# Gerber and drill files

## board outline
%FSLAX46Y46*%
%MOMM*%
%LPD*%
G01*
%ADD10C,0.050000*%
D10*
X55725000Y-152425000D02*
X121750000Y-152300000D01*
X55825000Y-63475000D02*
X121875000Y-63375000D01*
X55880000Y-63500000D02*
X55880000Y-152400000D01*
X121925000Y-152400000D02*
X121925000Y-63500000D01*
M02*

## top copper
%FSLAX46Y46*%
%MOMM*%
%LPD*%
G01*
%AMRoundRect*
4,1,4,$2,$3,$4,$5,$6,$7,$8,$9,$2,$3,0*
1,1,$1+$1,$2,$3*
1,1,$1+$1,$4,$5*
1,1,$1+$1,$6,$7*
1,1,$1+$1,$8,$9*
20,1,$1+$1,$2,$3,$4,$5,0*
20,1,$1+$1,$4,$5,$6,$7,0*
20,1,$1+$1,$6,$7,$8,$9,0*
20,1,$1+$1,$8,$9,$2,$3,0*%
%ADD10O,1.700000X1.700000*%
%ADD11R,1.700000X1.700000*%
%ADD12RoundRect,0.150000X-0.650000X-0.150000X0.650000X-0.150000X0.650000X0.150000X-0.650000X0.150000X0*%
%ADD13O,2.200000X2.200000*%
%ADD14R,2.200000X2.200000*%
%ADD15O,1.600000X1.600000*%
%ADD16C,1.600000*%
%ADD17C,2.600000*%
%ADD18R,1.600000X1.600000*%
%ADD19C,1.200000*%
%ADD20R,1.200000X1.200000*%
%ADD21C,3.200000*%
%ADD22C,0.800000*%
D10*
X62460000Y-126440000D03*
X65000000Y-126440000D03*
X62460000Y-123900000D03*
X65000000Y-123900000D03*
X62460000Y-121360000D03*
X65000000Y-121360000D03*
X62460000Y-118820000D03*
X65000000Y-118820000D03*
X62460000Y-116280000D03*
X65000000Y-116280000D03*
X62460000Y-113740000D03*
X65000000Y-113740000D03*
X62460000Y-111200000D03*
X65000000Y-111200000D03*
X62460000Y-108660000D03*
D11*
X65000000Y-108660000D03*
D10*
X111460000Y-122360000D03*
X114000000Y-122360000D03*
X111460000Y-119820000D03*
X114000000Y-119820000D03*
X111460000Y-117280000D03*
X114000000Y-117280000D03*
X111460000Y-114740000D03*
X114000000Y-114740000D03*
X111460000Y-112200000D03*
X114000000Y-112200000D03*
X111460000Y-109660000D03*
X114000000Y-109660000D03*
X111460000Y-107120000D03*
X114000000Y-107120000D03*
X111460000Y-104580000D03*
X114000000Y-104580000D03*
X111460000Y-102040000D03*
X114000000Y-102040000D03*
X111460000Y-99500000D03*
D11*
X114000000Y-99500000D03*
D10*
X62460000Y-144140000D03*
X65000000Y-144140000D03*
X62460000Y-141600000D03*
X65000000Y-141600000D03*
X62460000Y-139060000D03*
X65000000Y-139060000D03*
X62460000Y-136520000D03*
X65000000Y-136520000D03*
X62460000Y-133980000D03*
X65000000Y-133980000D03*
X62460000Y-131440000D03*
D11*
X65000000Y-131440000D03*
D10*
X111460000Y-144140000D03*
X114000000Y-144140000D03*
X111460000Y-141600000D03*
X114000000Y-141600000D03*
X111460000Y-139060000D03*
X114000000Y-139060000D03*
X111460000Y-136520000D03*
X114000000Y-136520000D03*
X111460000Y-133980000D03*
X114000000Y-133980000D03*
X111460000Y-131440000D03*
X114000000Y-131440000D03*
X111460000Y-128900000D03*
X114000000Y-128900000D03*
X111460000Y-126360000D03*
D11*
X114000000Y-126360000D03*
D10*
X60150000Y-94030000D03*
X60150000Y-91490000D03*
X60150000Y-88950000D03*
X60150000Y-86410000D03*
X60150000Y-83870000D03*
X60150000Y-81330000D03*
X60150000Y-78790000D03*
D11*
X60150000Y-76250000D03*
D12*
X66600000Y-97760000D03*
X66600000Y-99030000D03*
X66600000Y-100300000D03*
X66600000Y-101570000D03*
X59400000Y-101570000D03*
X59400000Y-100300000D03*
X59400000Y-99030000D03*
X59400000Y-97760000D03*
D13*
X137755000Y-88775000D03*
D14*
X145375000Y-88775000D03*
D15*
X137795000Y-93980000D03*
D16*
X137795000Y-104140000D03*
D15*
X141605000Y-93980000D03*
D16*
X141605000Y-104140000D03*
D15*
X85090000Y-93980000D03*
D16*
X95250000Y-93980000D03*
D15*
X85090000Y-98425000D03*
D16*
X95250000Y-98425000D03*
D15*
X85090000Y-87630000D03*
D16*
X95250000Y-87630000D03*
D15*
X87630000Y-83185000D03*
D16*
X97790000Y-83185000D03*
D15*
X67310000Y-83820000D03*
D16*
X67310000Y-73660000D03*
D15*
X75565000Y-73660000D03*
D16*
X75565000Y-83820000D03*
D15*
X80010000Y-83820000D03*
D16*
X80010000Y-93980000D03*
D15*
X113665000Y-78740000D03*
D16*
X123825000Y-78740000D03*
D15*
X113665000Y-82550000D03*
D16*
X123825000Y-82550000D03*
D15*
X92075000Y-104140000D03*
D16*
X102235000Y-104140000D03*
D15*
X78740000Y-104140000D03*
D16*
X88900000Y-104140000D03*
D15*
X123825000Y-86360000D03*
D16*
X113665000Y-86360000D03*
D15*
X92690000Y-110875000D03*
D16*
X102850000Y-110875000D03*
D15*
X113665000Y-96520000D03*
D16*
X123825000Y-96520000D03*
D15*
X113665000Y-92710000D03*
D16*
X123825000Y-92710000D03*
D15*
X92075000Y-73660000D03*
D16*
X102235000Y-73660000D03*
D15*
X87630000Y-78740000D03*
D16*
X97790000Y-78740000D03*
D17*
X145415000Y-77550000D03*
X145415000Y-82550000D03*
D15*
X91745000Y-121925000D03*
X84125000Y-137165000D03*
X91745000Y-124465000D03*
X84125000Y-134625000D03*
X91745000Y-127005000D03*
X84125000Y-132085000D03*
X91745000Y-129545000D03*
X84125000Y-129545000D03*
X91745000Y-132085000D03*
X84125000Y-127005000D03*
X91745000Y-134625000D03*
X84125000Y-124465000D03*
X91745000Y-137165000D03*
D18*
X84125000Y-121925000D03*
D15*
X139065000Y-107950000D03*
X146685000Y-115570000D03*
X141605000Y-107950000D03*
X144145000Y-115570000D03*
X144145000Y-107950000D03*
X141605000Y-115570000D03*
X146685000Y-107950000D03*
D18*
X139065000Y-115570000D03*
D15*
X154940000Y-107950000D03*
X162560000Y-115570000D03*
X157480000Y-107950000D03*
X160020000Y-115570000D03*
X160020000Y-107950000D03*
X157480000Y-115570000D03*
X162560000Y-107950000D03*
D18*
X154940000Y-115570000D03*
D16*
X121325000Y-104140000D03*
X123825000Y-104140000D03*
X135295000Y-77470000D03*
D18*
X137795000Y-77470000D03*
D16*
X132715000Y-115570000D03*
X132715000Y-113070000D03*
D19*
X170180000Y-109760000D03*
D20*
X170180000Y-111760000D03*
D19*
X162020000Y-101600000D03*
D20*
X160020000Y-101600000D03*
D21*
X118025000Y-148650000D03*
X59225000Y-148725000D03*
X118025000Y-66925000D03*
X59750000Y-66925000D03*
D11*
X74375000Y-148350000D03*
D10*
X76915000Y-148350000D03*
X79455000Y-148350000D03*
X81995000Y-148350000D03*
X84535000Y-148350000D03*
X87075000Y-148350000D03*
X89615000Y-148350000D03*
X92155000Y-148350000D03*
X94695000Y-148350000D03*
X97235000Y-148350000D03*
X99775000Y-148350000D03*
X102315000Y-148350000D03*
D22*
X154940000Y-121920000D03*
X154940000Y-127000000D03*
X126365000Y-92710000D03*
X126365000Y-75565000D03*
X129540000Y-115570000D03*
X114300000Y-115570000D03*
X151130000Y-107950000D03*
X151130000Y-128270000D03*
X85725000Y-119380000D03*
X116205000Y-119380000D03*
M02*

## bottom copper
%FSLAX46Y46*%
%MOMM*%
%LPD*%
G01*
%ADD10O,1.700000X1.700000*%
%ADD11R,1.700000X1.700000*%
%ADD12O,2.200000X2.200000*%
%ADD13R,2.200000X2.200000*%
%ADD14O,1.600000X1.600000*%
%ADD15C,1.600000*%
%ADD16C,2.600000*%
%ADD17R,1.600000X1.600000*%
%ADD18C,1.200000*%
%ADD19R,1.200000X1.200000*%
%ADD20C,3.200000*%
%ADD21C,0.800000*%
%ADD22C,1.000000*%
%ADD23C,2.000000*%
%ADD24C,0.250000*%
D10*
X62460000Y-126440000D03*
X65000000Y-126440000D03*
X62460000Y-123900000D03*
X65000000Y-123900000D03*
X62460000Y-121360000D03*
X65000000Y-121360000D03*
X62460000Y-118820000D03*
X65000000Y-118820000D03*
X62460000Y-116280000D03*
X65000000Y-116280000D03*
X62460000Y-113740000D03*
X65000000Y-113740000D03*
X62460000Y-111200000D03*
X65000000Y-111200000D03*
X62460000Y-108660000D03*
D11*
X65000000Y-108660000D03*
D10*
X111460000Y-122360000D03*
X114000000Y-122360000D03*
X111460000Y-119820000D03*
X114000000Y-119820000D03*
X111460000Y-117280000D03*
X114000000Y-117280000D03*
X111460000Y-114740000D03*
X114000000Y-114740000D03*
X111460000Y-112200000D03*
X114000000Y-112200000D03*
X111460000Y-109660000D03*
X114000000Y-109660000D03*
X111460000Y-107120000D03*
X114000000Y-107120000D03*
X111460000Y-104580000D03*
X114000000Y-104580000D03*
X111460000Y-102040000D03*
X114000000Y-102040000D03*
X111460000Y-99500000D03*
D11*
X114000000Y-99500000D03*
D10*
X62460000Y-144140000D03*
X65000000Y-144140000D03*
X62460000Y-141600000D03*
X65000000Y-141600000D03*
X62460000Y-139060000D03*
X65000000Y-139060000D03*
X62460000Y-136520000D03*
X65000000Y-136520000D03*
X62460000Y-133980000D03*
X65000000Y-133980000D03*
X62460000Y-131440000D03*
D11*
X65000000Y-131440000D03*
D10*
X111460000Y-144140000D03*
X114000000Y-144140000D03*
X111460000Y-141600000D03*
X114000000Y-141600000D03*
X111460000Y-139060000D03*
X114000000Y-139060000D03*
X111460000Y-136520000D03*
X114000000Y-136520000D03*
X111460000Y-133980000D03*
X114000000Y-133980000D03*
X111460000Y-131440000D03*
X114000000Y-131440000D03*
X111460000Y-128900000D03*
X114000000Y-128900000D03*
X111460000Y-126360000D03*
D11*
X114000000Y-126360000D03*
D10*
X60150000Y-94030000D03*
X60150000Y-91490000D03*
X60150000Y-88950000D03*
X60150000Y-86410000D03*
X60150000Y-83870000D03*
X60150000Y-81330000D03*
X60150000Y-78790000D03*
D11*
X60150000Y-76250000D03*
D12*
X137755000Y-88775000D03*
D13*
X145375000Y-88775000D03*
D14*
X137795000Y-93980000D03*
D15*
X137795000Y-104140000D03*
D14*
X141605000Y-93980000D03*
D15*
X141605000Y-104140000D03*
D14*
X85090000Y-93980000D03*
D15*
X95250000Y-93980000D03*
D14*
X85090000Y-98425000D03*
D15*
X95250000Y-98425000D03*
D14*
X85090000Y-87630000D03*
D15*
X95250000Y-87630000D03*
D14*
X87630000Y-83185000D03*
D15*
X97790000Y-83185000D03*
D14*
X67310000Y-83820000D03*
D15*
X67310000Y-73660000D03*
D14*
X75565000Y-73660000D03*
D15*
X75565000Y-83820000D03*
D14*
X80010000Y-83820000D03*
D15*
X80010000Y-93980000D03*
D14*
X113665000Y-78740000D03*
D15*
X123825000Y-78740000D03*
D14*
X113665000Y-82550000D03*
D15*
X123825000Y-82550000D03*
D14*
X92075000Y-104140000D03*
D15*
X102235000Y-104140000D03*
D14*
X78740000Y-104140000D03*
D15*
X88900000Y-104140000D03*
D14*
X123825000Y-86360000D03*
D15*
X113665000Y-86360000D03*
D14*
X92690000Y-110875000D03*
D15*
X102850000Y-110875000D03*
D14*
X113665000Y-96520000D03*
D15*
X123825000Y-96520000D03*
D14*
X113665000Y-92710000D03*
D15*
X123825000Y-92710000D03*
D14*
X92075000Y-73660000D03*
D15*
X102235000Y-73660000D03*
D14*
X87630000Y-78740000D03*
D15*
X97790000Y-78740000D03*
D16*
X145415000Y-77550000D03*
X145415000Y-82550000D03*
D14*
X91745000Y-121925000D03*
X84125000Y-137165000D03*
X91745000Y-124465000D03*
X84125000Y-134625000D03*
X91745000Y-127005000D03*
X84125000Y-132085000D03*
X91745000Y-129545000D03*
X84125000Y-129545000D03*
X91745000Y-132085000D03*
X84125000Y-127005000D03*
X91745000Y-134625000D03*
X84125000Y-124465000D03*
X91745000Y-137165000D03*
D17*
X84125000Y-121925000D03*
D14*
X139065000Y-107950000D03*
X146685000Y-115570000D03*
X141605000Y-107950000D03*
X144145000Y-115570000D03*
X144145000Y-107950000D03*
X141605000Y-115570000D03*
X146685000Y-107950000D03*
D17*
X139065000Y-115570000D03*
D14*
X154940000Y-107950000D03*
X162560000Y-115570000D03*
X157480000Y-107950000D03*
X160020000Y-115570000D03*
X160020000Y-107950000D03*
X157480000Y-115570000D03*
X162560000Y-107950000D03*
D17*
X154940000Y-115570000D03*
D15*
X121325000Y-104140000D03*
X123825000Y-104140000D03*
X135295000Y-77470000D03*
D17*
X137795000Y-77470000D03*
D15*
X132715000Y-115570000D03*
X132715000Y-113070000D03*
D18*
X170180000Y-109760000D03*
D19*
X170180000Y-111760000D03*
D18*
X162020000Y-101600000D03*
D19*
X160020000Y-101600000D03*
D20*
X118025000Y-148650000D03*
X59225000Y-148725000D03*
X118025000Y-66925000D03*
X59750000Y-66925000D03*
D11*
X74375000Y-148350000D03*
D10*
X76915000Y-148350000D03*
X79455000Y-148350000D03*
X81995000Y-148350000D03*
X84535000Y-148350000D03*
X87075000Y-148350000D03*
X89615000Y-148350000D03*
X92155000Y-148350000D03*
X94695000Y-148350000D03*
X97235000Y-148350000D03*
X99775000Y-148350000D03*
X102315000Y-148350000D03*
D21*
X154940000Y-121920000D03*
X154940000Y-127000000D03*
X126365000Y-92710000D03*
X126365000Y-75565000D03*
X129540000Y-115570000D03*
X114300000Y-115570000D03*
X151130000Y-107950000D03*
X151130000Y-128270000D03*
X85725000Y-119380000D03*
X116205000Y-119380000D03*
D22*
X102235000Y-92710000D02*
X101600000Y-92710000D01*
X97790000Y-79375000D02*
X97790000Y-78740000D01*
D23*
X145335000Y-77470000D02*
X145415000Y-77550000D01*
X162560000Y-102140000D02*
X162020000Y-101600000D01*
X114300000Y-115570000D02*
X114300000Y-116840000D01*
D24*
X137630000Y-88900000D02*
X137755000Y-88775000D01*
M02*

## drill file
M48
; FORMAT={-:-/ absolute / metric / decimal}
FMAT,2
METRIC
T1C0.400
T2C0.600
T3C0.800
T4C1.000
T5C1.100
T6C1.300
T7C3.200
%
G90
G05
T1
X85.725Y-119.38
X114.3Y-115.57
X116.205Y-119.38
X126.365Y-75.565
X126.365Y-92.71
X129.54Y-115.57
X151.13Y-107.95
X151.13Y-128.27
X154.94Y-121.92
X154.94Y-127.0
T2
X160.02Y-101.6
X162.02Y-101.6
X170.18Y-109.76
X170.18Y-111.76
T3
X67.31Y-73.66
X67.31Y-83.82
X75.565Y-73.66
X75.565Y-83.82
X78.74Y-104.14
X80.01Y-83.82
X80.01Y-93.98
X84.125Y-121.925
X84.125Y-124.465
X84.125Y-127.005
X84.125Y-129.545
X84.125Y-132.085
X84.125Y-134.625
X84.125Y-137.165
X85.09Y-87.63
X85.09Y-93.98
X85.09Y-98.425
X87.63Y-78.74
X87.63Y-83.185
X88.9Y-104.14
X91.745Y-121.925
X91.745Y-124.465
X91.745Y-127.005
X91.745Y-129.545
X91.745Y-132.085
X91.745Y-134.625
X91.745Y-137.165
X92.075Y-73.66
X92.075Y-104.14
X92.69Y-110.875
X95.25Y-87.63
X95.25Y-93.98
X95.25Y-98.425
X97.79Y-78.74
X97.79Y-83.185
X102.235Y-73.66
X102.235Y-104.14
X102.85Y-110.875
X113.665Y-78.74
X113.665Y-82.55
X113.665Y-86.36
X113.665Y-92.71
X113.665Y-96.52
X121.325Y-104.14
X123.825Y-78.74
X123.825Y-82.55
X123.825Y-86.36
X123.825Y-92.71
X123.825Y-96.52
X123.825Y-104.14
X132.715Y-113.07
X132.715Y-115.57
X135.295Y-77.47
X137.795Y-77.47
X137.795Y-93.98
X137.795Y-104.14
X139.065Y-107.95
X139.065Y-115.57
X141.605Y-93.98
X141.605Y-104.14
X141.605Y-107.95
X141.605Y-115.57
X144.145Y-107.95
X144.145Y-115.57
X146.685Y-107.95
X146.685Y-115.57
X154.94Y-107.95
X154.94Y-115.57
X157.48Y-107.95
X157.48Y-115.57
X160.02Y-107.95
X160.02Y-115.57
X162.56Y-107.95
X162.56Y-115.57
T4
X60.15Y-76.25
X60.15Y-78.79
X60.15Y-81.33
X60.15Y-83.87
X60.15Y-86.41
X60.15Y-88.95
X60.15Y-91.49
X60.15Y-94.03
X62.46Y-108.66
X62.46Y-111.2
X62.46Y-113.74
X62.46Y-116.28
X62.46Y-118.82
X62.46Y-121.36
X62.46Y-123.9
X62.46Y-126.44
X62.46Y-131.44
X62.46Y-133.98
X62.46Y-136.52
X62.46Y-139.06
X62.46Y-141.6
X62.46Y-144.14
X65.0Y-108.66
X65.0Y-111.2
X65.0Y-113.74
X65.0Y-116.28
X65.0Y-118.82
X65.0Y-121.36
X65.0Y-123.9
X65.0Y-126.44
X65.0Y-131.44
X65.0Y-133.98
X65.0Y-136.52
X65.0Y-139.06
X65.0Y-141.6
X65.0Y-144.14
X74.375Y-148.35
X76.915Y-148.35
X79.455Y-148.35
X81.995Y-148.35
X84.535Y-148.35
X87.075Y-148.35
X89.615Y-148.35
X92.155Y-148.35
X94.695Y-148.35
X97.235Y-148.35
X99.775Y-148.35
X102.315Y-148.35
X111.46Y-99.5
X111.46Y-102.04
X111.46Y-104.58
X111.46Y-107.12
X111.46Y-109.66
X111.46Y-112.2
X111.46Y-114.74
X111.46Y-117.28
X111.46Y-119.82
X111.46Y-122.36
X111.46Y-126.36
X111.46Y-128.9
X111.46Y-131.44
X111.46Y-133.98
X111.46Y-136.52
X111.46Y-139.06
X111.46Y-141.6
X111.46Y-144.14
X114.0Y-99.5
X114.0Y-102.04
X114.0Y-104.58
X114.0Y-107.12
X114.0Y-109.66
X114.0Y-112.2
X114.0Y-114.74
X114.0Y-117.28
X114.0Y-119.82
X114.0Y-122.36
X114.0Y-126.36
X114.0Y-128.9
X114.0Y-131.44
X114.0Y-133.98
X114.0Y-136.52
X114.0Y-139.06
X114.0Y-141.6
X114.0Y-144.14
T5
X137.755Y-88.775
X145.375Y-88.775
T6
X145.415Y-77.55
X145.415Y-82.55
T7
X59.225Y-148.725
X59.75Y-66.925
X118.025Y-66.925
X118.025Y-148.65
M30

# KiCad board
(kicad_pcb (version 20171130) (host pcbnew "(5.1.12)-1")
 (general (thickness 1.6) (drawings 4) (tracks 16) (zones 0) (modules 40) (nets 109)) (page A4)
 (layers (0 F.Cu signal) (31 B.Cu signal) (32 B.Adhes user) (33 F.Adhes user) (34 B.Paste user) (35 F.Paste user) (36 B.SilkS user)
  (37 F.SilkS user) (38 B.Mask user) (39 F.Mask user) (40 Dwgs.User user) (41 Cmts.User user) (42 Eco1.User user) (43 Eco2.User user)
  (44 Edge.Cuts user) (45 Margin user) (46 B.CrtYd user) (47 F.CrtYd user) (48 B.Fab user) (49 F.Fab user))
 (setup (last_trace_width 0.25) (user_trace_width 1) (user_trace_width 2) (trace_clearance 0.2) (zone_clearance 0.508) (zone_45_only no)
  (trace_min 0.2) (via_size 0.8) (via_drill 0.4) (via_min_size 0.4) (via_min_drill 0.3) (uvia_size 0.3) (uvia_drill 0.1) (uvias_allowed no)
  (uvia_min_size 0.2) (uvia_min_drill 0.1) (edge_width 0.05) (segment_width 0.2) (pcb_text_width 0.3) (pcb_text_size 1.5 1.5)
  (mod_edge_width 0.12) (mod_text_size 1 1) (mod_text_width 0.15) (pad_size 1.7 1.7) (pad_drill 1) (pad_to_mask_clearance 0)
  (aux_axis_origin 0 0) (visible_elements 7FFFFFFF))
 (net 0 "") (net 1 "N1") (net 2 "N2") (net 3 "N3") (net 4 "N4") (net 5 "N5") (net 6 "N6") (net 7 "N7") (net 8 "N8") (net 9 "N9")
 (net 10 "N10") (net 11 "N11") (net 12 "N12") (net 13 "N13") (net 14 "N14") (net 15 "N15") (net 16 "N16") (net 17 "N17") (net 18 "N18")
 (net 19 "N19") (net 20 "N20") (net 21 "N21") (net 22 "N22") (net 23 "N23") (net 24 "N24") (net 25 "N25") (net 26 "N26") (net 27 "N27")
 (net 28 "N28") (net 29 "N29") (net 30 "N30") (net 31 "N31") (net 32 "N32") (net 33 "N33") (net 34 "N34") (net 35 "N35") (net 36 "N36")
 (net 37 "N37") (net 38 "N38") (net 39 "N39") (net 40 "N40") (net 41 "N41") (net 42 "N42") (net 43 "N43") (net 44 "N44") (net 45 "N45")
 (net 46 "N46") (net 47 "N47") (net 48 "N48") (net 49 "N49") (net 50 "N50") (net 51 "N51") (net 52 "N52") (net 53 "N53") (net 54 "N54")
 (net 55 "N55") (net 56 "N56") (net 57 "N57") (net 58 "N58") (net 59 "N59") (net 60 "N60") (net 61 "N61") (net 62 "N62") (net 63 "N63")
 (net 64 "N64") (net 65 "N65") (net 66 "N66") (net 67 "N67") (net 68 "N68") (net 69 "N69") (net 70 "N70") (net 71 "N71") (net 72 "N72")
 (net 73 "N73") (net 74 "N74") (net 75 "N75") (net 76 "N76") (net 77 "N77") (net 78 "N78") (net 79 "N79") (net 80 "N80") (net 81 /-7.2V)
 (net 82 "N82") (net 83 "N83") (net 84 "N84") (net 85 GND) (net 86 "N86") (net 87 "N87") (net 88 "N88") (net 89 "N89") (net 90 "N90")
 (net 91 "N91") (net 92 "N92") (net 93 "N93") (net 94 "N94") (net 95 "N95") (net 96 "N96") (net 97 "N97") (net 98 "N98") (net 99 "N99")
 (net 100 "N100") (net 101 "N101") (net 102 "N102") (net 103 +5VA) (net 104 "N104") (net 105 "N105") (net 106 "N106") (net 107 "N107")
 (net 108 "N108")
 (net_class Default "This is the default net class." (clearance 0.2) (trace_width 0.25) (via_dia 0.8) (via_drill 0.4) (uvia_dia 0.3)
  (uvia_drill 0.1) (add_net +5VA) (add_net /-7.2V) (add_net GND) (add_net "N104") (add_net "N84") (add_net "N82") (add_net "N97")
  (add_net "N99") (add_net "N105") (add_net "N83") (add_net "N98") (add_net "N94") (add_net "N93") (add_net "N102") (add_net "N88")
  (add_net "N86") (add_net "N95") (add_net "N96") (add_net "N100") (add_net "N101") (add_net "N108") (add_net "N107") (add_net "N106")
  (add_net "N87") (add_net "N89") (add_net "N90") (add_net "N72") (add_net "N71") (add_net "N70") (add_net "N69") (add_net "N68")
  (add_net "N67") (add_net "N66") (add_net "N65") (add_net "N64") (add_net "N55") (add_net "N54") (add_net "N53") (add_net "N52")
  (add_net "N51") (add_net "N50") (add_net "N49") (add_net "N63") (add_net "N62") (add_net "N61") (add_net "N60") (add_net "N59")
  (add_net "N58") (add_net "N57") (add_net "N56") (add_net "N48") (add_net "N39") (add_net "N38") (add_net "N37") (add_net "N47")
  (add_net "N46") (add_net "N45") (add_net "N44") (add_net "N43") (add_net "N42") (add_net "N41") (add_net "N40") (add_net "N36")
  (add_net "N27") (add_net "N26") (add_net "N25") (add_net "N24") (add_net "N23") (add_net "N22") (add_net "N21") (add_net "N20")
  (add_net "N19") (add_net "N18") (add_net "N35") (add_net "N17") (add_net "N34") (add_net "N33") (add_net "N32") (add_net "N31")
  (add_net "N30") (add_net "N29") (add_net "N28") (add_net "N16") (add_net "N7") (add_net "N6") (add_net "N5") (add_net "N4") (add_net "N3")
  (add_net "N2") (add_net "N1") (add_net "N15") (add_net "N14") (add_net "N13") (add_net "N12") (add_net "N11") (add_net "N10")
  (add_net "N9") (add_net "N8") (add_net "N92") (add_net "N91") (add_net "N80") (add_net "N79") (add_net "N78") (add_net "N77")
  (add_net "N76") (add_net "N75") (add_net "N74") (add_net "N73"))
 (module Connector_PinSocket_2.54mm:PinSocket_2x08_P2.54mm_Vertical (layer F.Cu) (at 65 108.66)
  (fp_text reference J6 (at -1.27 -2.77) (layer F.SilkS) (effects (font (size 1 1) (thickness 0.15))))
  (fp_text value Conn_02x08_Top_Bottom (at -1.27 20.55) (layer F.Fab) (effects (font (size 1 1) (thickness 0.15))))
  (pad 16 thru_hole oval (at -2.54 17.78) (size 1.7 1.7) (drill 1) (layers *.Cu *.Mask) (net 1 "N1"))
  (pad 15 thru_hole oval (at 0 17.78) (size 1.7 1.7) (drill 1) (layers *.Cu *.Mask) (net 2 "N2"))
  (pad 14 thru_hole oval (at -2.54 15.24) (size 1.7 1.7) (drill 1) (layers *.Cu *.Mask) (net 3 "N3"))
  (pad 13 thru_hole oval (at 0 15.24) (size 1.7 1.7) (drill 1) (layers *.Cu *.Mask) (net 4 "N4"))
  (pad 12 thru_hole oval (at -2.54 12.7) (size 1.7 1.7) (drill 1) (layers *.Cu *.Mask) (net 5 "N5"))
  (pad 11 thru_hole oval (at 0 12.7) (size 1.7 1.7) (drill 1) (layers *.Cu *.Mask) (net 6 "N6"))
  (pad 10 thru_hole oval (at -2.54 10.16) (size 1.7 1.7) (drill 1) (layers *.Cu *.Mask) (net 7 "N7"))
  (pad 9 thru_hole oval (at 0 10.16) (size 1.7 1.7) (drill 1) (layers *.Cu *.Mask) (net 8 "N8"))
  (pad 8 thru_hole oval (at -2.54 7.62) (size 1.7 1.7) (drill 1) (layers *.Cu *.Mask) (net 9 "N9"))
  (pad 7 thru_hole oval (at 0 7.62) (size 1.7 1.7) (drill 1) (layers *.Cu *.Mask) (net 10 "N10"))
  (pad 6 thru_hole oval (at -2.54 5.08) (size 1.7 1.7) (drill 1) (layers *.Cu *.Mask) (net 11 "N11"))
  (pad 5 thru_hole oval (at 0 5.08) (size 1.7 1.7) (drill 1) (layers *.Cu *.Mask) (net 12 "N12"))
  (pad 4 thru_hole oval (at -2.54 2.54) (size 1.7 1.7) (drill 1) (layers *.Cu *.Mask) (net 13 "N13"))
  (pad 3 thru_hole oval (at 0 2.54) (size 1.7 1.7) (drill 1) (layers *.Cu *.Mask) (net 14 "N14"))
  (pad 2 thru_hole oval (at -2.54 0) (size 1.7 1.7) (drill 1) (layers *.Cu *.Mask) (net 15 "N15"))
  (pad 1 thru_hole rect (at 0 0) (size 1.7 1.7) (drill 1) (layers *.Cu *.Mask) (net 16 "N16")))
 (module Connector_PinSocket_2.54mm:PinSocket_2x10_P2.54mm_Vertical (layer F.Cu) (at 114 99.5)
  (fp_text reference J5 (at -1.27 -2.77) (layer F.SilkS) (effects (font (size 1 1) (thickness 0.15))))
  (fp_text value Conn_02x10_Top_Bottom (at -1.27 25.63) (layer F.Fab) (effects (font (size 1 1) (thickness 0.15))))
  (pad 20 thru_hole oval (at -2.54 22.86) (size 1.7 1.7) (drill 1) (layers *.Cu *.Mask) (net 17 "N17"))
  (pad 19 thru_hole oval (at 0 22.86) (size 1.7 1.7) (drill 1) (layers *.Cu *.Mask) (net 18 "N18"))
  (pad 18 thru_hole oval (at -2.54 20.32) (size 1.7 1.7) (drill 1) (layers *.Cu *.Mask) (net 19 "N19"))
  (pad 17 thru_hole oval (at 0 20.32) (size 1.7 1.7) (drill 1) (layers *.Cu *.Mask) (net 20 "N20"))
  (pad 16 thru_hole oval (at -2.54 17.78) (size 1.7 1.7) (drill 1) (layers *.Cu *.Mask) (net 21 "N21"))
  (pad 15 thru_hole oval (at 0 17.78) (size 1.7 1.7) (drill 1) (layers *.Cu *.Mask) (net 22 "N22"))
  (pad 14 thru_hole oval (at -2.54 15.24) (size 1.7 1.7) (drill 1) (layers *.Cu *.Mask) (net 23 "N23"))
  (pad 13 thru_hole oval (at 0 15.24) (size 1.7 1.7) (drill 1) (layers *.Cu *.Mask) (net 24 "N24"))
  (pad 12 thru_hole oval (at -2.54 12.7) (size 1.7 1.7) (drill 1) (layers *.Cu *.Mask) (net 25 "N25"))
  (pad 11 thru_hole oval (at 0 12.7) (size 1.7 1.7) (drill 1) (layers *.Cu *.Mask) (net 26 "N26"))
  (pad 10 thru_hole oval (at -2.54 10.16) (size 1.7 1.7) (drill 1) (layers *.Cu *.Mask) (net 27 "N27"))
  (pad 9 thru_hole oval (at 0 10.16) (size 1.7 1.7) (drill 1) (layers *.Cu *.Mask) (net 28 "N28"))
  (pad 8 thru_hole oval (at -2.54 7.62) (size 1.7 1.7) (drill 1) (layers *.Cu *.Mask) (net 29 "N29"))
  (pad 7 thru_hole oval (at 0 7.62) (size 1.7 1.7) (drill 1) (layers *.Cu *.Mask) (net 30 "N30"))
  (pad 6 thru_hole oval (at -2.54 5.08) (size 1.7 1.7) (drill 1) (layers *.Cu *.Mask) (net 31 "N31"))
  (pad 5 thru_hole oval (at 0 5.08) (size 1.7 1.7) (drill 1) (layers *.Cu *.Mask) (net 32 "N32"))
  (pad 4 thru_hole oval (at -2.54 2.54) (size 1.7 1.7) (drill 1) (layers *.Cu *.Mask) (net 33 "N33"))
  (pad 3 thru_hole oval (at 0 2.54) (size 1.7 1.7) (drill 1) (layers *.Cu *.Mask) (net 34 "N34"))
  (pad 2 thru_hole oval (at -2.54 0) (size 1.7 1.7) (drill 1) (layers *.Cu *.Mask) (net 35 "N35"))
  (pad 1 thru_hole rect (at 0 0) (size 1.7 1.7) (drill 1) (layers *.Cu *.Mask) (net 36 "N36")))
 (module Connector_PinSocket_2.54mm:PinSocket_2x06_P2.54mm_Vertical (layer F.Cu) (at 65 131.44)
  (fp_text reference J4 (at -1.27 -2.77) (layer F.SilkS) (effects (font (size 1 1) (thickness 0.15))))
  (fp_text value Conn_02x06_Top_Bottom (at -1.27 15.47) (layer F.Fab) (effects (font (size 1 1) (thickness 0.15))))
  (pad 12 thru_hole oval (at -2.54 12.7) (size 1.7 1.7) (drill 1) (layers *.Cu *.Mask) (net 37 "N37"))
  (pad 11 thru_hole oval (at 0 12.7) (size 1.7 1.7) (drill 1) (layers *.Cu *.Mask) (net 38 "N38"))
  (pad 10 thru_hole oval (at -2.54 10.16) (size 1.7 1.7) (drill 1) (layers *.Cu *.Mask) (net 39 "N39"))
  (pad 9 thru_hole oval (at 0 10.16) (size 1.7 1.7) (drill 1) (layers *.Cu *.Mask) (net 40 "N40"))
  (pad 8 thru_hole oval (at -2.54 7.62) (size 1.7 1.7) (drill 1) (layers *.Cu *.Mask) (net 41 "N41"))
  (pad 7 thru_hole oval (at 0 7.62) (size 1.7 1.7) (drill 1) (layers *.Cu *.Mask) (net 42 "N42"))
  (pad 6 thru_hole oval (at -2.54 5.08) (size 1.7 1.7) (drill 1) (layers *.Cu *.Mask) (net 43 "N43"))
  (pad 5 thru_hole oval (at 0 5.08) (size 1.7 1.7) (drill 1) (layers *.Cu *.Mask) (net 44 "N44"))
  (pad 4 thru_hole oval (at -2.54 2.54) (size 1.7 1.7) (drill 1) (layers *.Cu *.Mask) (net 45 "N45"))
  (pad 3 thru_hole oval (at 0 2.54) (size 1.7 1.7) (drill 1) (layers *.Cu *.Mask) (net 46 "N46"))
  (pad 2 thru_hole oval (at -2.54 0) (size 1.7 1.7) (drill 1) (layers *.Cu *.Mask) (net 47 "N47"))
  (pad 1 thru_hole rect (at 0 0) (size 1.7 1.7) (drill 1) (layers *.Cu *.Mask) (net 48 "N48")))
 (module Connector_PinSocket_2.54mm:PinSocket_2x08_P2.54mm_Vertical (layer F.Cu) (at 114 126.36)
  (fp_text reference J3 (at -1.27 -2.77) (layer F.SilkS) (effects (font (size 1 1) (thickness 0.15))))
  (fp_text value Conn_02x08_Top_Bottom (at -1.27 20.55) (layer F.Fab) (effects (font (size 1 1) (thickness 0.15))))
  (pad 16 thru_hole oval (at -2.54 17.78) (size 1.7 1.7) (drill 1) (layers *.Cu *.Mask) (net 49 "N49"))
  (pad 15 thru_hole oval (at 0 17.78) (size 1.7 1.7) (drill 1) (layers *.Cu *.Mask) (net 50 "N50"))
  (pad 14 thru_hole oval (at -2.54 15.24) (size 1.7 1.7) (drill 1) (layers *.Cu *.Mask) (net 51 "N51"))
  (pad 13 thru_hole oval (at 0 15.24) (size 1.7 1.7) (drill 1) (layers *.Cu *.Mask) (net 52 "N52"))
  (pad 12 thru_hole oval (at -2.54 12.7) (size 1.7 1.7) (drill 1) (layers *.Cu *.Mask) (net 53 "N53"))
  (pad 11 thru_hole oval (at 0 12.7) (size 1.7 1.7) (drill 1) (layers *.Cu *.Mask) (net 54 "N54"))
  (pad 10 thru_hole oval (at -2.54 10.16) (size 1.7 1.7) (drill 1) (layers *.Cu *.Mask) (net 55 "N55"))
  (pad 9 thru_hole oval (at 0 10.16) (size 1.7 1.7) (drill 1) (layers *.Cu *.Mask) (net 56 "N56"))
  (pad 8 thru_hole oval (at -2.54 7.62) (size 1.7 1.7) (drill 1) (layers *.Cu *.Mask) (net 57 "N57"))
  (pad 7 thru_hole oval (at 0 7.62) (size 1.7 1.7) (drill 1) (layers *.Cu *.Mask) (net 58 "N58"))
  (pad 6 thru_hole oval (at -2.54 5.08) (size 1.7 1.7) (drill 1) (layers *.Cu *.Mask) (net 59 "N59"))
  (pad 5 thru_hole oval (at 0 5.08) (size 1.7 1.7) (drill 1) (layers *.Cu *.Mask) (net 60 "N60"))
  (pad 4 thru_hole oval (at -2.54 2.54) (size 1.7 1.7) (drill 1) (layers *.Cu *.Mask) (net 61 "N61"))
  (pad 3 thru_hole oval (at 0 2.54) (size 1.7 1.7) (drill 1) (layers *.Cu *.Mask) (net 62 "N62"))
  (pad 2 thru_hole oval (at -2.54 0) (size 1.7 1.7) (drill 1) (layers *.Cu *.Mask) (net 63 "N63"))
  (pad 1 thru_hole rect (at 0 0) (size 1.7 1.7) (drill 1) (layers *.Cu *.Mask) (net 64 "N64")))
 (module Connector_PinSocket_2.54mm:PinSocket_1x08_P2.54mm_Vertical (layer F.Cu) (at 60.15 76.25)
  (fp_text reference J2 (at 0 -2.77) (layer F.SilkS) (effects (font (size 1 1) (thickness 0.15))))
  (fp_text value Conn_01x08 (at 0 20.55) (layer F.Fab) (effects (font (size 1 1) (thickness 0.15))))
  (pad 8 thru_hole oval (at 0 17.78) (size 1.7 1.7) (drill 1) (layers *.Cu *.Mask) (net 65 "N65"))
  (pad 7 thru_hole oval (at 0 15.24) (size 1.7 1.7) (drill 1) (layers *.Cu *.Mask) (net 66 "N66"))
  (pad 6 thru_hole oval (at 0 12.7) (size 1.7 1.7) (drill 1) (layers *.Cu *.Mask) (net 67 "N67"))
  (pad 5 thru_hole oval (at 0 10.16) (size 1.7 1.7) (drill 1) (layers *.Cu *.Mask) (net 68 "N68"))
  (pad 4 thru_hole oval (at 0 7.62) (size 1.7 1.7) (drill 1) (layers *.Cu *.Mask) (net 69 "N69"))
  (pad 3 thru_hole oval (at 0 5.08) (size 1.7 1.7) (drill 1) (layers *.Cu *.Mask) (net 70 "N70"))
  (pad 2 thru_hole oval (at 0 2.54) (size 1.7 1.7) (drill 1) (layers *.Cu *.Mask) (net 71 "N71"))
  (pad 1 thru_hole rect (at 0 0) (size 1.7 1.7) (drill 1) (layers *.Cu *.Mask) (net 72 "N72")))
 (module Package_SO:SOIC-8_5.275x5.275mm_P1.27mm (layer F.Cu) (at 63 99.665)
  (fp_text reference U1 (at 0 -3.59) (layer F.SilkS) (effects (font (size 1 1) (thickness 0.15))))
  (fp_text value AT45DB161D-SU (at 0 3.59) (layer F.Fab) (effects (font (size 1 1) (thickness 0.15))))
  (pad 8 smd roundrect (at 3.6 -1.905) (size 1.6 0.6) (layers F.Cu F.Paste F.Mask) (roundrect_rratio 0.25) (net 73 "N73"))
  (pad 7 smd roundrect (at 3.6 -0.635) (size 1.6 0.6) (layers F.Cu F.Paste F.Mask) (roundrect_rratio 0.25) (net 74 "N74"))
  (pad 6 smd roundrect (at 3.6 0.635) (size 1.6 0.6) (layers F.Cu F.Paste F.Mask) (roundrect_rratio 0.25) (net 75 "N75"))
  (pad 5 smd roundrect (at 3.6 1.905) (size 1.6 0.6) (layers F.Cu F.Paste F.Mask) (roundrect_rratio 0.25) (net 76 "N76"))
  (pad 4 smd roundrect (at -3.6 1.905) (size 1.6 0.6) (layers F.Cu F.Paste F.Mask) (roundrect_rratio 0.25) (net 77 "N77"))
  (pad 3 smd roundrect (at -3.6 0.635) (size 1.6 0.6) (layers F.Cu F.Paste F.Mask) (roundrect_rratio 0.25) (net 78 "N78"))
  (pad 2 smd roundrect (at -3.6 -0.635) (size 1.6 0.6) (layers F.Cu F.Paste F.Mask) (roundrect_rratio 0.25) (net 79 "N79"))
  (pad 1 smd roundrect (at -3.6 -1.905) (size 1.6 0.6) (layers F.Cu F.Paste F.Mask) (roundrect_rratio 0.25) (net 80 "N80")))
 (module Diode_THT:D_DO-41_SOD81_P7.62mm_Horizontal (layer F.Cu) (at 145.375 88.775 180)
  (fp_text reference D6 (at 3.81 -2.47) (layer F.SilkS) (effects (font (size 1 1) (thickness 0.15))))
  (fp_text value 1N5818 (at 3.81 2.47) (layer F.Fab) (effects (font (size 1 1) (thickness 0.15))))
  (pad 2 thru_hole oval (at 7.62 0 180) (size 2.2 2.2) (drill 1.1) (layers *.Cu *.Mask) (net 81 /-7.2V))
  (pad 1 thru_hole rect (at 0 0 180) (size 2.2 2.2) (drill 1.1) (layers *.Cu *.Mask) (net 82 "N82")))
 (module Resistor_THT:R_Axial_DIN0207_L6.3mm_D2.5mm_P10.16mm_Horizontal (layer F.Cu) (at 137.795 104.14 90)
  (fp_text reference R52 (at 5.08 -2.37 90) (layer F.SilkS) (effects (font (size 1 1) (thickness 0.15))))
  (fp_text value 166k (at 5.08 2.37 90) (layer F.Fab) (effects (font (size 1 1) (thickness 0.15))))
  (pad 2 thru_hole oval (at 10.16 0 90) (size 1.6 1.6) (drill 0.8) (layers *.Cu *.Mask) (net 81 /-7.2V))
  (pad 1 thru_hole circle (at 0 0 90) (size 1.6 1.6) (drill 0.8) (layers *.Cu *.Mask) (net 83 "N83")))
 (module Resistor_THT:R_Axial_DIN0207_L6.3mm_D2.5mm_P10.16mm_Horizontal (layer F.Cu) (at 141.605 104.14 90)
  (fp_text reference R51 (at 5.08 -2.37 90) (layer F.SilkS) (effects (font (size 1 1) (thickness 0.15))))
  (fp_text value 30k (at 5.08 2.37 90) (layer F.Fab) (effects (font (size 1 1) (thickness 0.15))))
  (pad 2 thru_hole oval (at 10.16 0 90) (size 1.6 1.6) (drill 0.8) (layers *.Cu *.Mask) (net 83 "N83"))
  (pad 1 thru_hole circle (at 0 0 90) (size 1.6 1.6) (drill 0.8) (layers *.Cu *.Mask) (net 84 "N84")))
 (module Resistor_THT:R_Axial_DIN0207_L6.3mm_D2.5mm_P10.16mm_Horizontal (layer F.Cu) (at 95.25 93.98 180)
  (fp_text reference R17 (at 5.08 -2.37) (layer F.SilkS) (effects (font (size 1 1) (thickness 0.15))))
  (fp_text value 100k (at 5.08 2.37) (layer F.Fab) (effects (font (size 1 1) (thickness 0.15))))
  (pad 2 thru_hole oval (at 10.16 0 180) (size 1.6 1.6) (drill 0.8) (layers *.Cu *.Mask) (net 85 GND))
  (pad 1 thru_hole circle (at 0 0 180) (size 1.6 1.6) (drill 0.8) (layers *.Cu *.Mask) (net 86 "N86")))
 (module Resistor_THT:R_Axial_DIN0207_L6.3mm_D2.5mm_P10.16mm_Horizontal (layer F.Cu) (at 95.25 98.425 180)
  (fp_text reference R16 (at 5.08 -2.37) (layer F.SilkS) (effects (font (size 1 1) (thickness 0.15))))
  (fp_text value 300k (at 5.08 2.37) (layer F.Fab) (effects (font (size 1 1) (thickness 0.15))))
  (pad 2 thru_hole oval (at 10.16 0 180) (size 1.6 1.6) (drill 0.8) (layers *.Cu *.Mask) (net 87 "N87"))
  (pad 1 thru_hole circle (at 0 0 180) (size 1.6 1.6) (drill 0.8) (layers *.Cu *.Mask) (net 86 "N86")))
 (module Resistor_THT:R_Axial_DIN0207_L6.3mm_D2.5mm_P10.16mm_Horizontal (layer F.Cu) (at 95.25 87.63 180)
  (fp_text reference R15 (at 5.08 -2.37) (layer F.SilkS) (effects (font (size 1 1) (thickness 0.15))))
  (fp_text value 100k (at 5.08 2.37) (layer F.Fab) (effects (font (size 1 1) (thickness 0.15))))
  (pad 2 thru_hole oval (at 10.16 0 180) (size 1.6 1.6) (drill 0.8) (layers *.Cu *.Mask) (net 85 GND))
  (pad 1 thru_hole circle (at 0 0 180) (size 1.6 1.6) (drill 0.8) (layers *.Cu *.Mask) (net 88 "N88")))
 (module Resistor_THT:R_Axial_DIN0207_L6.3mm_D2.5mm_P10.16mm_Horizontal (layer F.Cu) (at 97.79 83.185 180)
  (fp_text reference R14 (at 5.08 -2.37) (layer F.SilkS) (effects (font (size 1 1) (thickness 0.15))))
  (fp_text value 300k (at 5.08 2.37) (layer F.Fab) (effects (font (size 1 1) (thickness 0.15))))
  (pad 2 thru_hole oval (at 10.16 0 180) (size 1.6 1.6) (drill 0.8) (layers *.Cu *.Mask) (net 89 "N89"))
  (pad 1 thru_hole circle (at 0 0 180) (size 1.6 1.6) (drill 0.8) (layers *.Cu *.Mask) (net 88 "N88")))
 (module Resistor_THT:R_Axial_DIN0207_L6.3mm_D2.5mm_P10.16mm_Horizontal (layer F.Cu) (at 67.31 73.66 270)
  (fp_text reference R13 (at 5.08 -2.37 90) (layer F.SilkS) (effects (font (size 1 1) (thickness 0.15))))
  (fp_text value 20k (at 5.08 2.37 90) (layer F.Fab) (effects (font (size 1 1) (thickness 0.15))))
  (pad 2 thru_hole oval (at 10.16 0 270) (size 1.6 1.6) (drill 0.8) (layers *.Cu *.Mask) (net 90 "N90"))
  (pad 1 thru_hole circle (at 0 0 270) (size 1.6 1.6) (drill 0.8) (layers *.Cu *.Mask) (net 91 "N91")))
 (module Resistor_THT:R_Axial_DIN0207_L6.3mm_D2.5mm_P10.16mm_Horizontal (layer F.Cu) (at 75.565 83.82 90)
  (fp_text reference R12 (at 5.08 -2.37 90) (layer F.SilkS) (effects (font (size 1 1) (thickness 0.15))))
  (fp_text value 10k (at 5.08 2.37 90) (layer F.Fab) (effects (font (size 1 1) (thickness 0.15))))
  (pad 2 thru_hole oval (at 10.16 0 90) (size 1.6 1.6) (drill 0.8) (layers *.Cu *.Mask) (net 91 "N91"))
  (pad 1 thru_hole circle (at 0 0 90) (size 1.6 1.6) (drill 0.8) (layers *.Cu *.Mask) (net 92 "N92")))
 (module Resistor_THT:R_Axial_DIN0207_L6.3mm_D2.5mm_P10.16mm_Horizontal (layer F.Cu) (at 80.01 93.98 90)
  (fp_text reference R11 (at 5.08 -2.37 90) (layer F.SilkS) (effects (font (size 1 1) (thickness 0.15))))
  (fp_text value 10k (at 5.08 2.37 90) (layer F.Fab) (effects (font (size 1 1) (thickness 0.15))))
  (pad 2 thru_hole oval (at 10.16 0 90) (size 1.6 1.6) (drill 0.8) (layers *.Cu *.Mask) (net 92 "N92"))
  (pad 1 thru_hole circle (at 0 0 90) (size 1.6 1.6) (drill 0.8) (layers *.Cu *.Mask) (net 85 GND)))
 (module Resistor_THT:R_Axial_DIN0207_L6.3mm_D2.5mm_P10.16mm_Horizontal (layer F.Cu) (at 123.825 78.74 180)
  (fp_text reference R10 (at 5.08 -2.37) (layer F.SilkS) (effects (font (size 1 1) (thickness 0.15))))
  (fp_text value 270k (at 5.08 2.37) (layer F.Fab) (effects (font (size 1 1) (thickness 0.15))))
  (pad 2 thru_hole oval (at 10.16 0 180) (size 1.6 1.6) (drill 0.8) (layers *.Cu *.Mask) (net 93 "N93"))
  (pad 1 thru_hole circle (at 0 0 180) (size 1.6 1.6) (drill 0.8) (layers *.Cu *.Mask) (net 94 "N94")))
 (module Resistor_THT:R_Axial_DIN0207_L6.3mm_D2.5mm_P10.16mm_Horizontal (layer F.Cu) (at 123.825 82.55 180)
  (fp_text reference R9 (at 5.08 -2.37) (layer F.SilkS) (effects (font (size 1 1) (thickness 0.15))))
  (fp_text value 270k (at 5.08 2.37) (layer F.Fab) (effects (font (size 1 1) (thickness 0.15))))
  (pad 2 thru_hole oval (at 10.16 0 180) (size 1.6 1.6) (drill 0.8) (layers *.Cu *.Mask) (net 94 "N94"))
  (pad 1 thru_hole circle (at 0 0 180) (size 1.6 1.6) (drill 0.8) (layers *.Cu *.Mask) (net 91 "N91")))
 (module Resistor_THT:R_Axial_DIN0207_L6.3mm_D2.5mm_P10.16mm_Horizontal (layer F.Cu) (at 102.235 104.14 180)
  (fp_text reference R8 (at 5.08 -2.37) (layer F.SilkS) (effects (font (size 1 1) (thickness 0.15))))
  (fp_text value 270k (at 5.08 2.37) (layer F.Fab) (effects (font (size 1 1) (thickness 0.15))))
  (pad 2 thru_hole oval (at 10.16 0 180) (size 1.6 1.6) (drill 0.8) (layers *.Cu *.Mask) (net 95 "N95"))
  (pad 1 thru_hole circle (at 0 0 180) (size 1.6 1.6) (drill 0.8) (layers *.Cu *.Mask) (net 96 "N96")))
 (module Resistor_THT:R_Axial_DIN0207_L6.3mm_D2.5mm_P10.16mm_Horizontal (layer F.Cu) (at 88.9 104.14 180)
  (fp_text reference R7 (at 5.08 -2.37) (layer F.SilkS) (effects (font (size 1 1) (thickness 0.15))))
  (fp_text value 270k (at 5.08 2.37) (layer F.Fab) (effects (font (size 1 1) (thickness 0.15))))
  (pad 2 thru_hole oval (at 10.16 0 180) (size 1.6 1.6) (drill 0.8) (layers *.Cu *.Mask) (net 92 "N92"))
  (pad 1 thru_hole circle (at 0 0 180) (size 1.6 1.6) (drill 0.8) (layers *.Cu *.Mask) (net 95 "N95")))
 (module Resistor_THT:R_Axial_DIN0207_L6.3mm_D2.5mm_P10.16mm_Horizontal (layer F.Cu) (at 113.665 86.36)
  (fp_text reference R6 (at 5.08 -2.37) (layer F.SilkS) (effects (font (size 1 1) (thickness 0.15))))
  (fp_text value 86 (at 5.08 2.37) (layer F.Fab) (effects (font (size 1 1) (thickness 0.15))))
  (pad 2 thru_hole oval (at 10.16 0) (size 1.6 1.6) (drill 0.8) (layers *.Cu *.Mask) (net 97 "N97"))
  (pad 1 thru_hole circle (at 0 0) (size 1.6 1.6) (drill 0.8) (layers *.Cu *.Mask) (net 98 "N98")))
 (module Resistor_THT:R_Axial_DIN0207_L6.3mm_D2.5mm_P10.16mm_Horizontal (layer F.Cu) (at 102.85 110.875 180)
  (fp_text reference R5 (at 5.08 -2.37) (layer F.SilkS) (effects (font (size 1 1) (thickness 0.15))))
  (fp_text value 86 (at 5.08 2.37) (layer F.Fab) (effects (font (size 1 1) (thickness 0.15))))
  (pad 2 thru_hole oval (at 10.16 0 180) (size 1.6 1.6) (drill 0.8) (layers *.Cu *.Mask) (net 96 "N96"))
  (pad 1 thru_hole circle (at 0 0 180) (size 1.6 1.6) (drill 0.8) (layers *.Cu *.Mask) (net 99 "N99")))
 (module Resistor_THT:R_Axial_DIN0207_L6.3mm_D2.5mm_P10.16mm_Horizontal (layer F.Cu) (at 123.825 96.52 180)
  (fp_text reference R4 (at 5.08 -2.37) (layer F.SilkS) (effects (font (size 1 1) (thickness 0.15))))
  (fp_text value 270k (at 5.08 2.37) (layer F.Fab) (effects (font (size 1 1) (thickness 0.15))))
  (pad 2 thru_hole oval (at 10.16 0 180) (size 1.6 1.6) (drill 0.8) (layers *.Cu *.Mask) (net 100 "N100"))
  (pad 1 thru_hole circle (at 0 0 180) (size 1.6 1.6) (drill 0.8) (layers *.Cu *.Mask) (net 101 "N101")))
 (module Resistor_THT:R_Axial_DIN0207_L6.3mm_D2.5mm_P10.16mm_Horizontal (layer F.Cu) (at 123.825 92.71 180)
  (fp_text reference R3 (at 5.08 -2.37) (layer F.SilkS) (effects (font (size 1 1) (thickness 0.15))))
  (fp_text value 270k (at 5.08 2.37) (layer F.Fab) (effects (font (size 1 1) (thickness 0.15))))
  (pad 2 thru_hole oval (at 10.16 0 180) (size 1.6 1.6) (drill 0.8) (layers *.Cu *.Mask) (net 101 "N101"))
  (pad 1 thru_hole circle (at 0 0 180) (size 1.6 1.6) (drill 0.8) (layers *.Cu *.Mask) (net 93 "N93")))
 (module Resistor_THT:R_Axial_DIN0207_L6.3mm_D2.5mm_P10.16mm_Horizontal (layer F.Cu) (at 102.235 73.66 180)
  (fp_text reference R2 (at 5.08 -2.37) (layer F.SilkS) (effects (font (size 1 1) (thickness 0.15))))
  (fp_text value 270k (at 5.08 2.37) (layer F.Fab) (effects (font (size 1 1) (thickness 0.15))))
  (pad 2 thru_hole oval (at 10.16 0 180) (size 1.6 1.6) (drill 0.8) (layers *.Cu *.Mask) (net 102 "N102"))
  (pad 1 thru_hole circle (at 0 0 180) (size 1.6 1.6) (drill 0.8) (layers *.Cu *.Mask) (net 98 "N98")))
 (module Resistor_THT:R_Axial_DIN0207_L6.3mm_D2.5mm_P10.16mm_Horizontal (layer F.Cu) (at 97.79 78.74 180)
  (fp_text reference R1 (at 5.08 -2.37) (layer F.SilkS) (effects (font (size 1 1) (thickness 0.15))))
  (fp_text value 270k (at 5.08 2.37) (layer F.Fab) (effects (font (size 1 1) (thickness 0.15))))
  (pad 2 thru_hole oval (at 10.16 0 180) (size 1.6 1.6) (drill 0.8) (layers *.Cu *.Mask) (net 92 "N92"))
  (pad 1 thru_hole circle (at 0 0 180) (size 1.6 1.6) (drill 0.8) (layers *.Cu *.Mask) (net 102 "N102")))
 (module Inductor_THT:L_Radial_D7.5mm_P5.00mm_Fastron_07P (layer F.Cu) (at 145.415 82.55 90)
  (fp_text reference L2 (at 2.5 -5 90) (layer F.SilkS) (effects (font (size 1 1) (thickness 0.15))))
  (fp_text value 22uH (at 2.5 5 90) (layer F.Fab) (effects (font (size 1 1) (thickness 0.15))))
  (pad 2 thru_hole circle (at 5 0 90) (size 2.6 2.6) (drill 1.3) (layers *.Cu *.Mask) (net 85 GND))
  (pad 1 thru_hole circle (at 0 0 90) (size 2.6 2.6) (drill 1.3) (layers *.Cu *.Mask) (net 82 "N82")))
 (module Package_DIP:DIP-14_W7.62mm (layer F.Cu) (at 84.125 121.925)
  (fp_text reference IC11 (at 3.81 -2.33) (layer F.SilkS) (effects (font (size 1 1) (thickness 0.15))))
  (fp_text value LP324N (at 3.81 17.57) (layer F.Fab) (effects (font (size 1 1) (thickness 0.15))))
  (pad 14 thru_hole oval (at 7.62 0) (size 1.6 1.6) (drill 0.8) (layers *.Cu *.Mask) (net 93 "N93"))
  (pad 7 thru_hole oval (at 0 15.24) (size 1.6 1.6) (drill 0.8) (layers *.Cu *.Mask) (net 96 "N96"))
  (pad 13 thru_hole oval (at 7.62 2.54) (size 1.6 1.6) (drill 0.8) (layers *.Cu *.Mask) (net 94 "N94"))
  (pad 6 thru_hole oval (at 0 12.7) (size 1.6 1.6) (drill 0.8) (layers *.Cu *.Mask) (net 95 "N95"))
  (pad 12 thru_hole oval (at 7.62 5.08) (size 1.6 1.6) (drill 0.8) (layers *.Cu *.Mask) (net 98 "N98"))
  (pad 5 thru_hole oval (at 0 10.16) (size 1.6 1.6) (drill 0.8) (layers *.Cu *.Mask) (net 86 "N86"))
  (pad 11 thru_hole oval (at 7.62 7.62) (size 1.6 1.6) (drill 0.8) (layers *.Cu *.Mask) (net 81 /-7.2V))
  (pad 4 thru_hole oval (at 0 7.62) (size 1.6 1.6) (drill 0.8) (layers *.Cu *.Mask) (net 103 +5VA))
  (pad 10 thru_hole oval (at 7.62 10.16) (size 1.6 1.6) (drill 0.8) (layers *.Cu *.Mask) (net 97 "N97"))
  (pad 3 thru_hole oval (at 0 5.08) (size 1.6 1.6) (drill 0.8) (layers *.Cu *.Mask) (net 88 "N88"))
  (pad 9 thru_hole oval (at 7.62 12.7) (size 1.6 1.6) (drill 0.8) (layers *.Cu *.Mask) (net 101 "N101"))
  (pad 2 thru_hole oval (at 0 2.54) (size 1.6 1.6) (drill 0.8) (layers *.Cu *.Mask) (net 102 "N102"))
  (pad 8 thru_hole oval (at 7.62 15.24) (size 1.6 1.6) (drill 0.8) (layers *.Cu *.Mask) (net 100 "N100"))
  (pad 1 thru_hole rect (at 0 0) (size 1.6 1.6) (drill 0.8) (layers *.Cu *.Mask) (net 98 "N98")))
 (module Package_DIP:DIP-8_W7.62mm (layer F.Cu) (at 139.065 115.57 90)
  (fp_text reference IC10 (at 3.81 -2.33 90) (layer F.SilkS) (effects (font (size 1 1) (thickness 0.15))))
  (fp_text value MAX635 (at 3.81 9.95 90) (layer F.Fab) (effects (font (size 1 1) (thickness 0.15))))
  (pad 8 thru_hole oval (at 7.62 0 90) (size 1.6 1.6) (drill 0.8) (layers *.Cu *.Mask) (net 83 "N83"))
  (pad 4 thru_hole oval (at 0 7.62 90) (size 1.6 1.6) (drill 0.8) (layers *.Cu *.Mask) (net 85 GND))
  (pad 7 thru_hole oval (at 7.62 2.54 90) (size 1.6 1.6) (drill 0.8) (layers *.Cu *.Mask) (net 84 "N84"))
  (pad 3 thru_hole oval (at 0 5.08 90) (size 1.6 1.6) (drill 0.8) (layers *.Cu *.Mask) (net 85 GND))
  (pad 6 thru_hole oval (at 7.62 5.08 90) (size 1.6 1.6) (drill 0.8) (layers *.Cu *.Mask) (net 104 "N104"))
  (pad 2 thru_hole oval (at 0 2.54 90) (size 1.6 1.6) (drill 0.8) (layers *.Cu *.Mask) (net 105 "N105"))
  (pad 5 thru_hole oval (at 7.62 7.62 90) (size 1.6 1.6) (drill 0.8) (layers *.Cu *.Mask) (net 82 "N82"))
  (pad 1 thru_hole rect (at 0 0 90) (size 1.6 1.6) (drill 0.8) (layers *.Cu *.Mask) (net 85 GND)))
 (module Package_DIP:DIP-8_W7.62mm (layer F.Cu) (at 154.94 115.57 90)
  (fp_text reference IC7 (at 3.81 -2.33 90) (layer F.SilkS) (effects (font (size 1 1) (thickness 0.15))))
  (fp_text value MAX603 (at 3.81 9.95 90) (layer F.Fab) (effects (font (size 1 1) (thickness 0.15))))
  (pad 8 thru_hole oval (at 7.62 0 90) (size 1.6 1.6) (drill 0.8) (layers *.Cu *.Mask) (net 103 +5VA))
  (pad 4 thru_hole oval (at 0 7.62 90) (size 1.6 1.6) (drill 0.8) (layers *.Cu *.Mask) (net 104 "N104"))
  (pad 7 thru_hole oval (at 7.62 2.54 90) (size 1.6 1.6) (drill 0.8) (layers *.Cu *.Mask) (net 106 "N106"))
  (pad 3 thru_hole oval (at 0 5.08 90) (size 1.6 1.6) (drill 0.8) (layers *.Cu *.Mask) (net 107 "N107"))
  (pad 6 thru_hole oval (at 7.62 5.08 90) (size 1.6 1.6) (drill 0.8) (layers *.Cu *.Mask) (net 85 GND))
  (pad 2 thru_hole oval (at 0 2.54 90) (size 1.6 1.6) (drill 0.8) (layers *.Cu *.Mask) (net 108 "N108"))
  (pad 5 thru_hole oval (at 7.62 7.62 90) (size 1.6 1.6) (drill 0.8) (layers *.Cu *.Mask) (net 85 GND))
  (pad 1 thru_hole rect (at 0 0 90) (size 1.6 1.6) (drill 0.8) (layers *.Cu *.Mask) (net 104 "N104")))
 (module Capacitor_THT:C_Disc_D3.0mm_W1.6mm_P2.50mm (layer F.Cu) (at 123.825 104.14 180)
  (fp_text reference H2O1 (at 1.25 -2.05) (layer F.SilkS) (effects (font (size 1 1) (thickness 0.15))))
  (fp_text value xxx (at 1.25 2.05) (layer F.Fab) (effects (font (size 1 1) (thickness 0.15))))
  (pad 2 thru_hole circle (at 2.5 0 180) (size 1.6 1.6) (drill 0.8) (layers *.Cu *.Mask) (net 99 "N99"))
  (pad 1 thru_hole circle (at 0 0 180) (size 1.6 1.6) (drill 0.8) (layers *.Cu *.Mask) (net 97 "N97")))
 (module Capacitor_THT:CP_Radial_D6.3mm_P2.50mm (layer F.Cu) (at 137.795 77.47 180)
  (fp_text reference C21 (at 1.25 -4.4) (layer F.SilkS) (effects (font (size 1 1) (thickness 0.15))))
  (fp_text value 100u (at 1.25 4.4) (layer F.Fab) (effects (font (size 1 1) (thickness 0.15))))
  (pad 2 thru_hole circle (at 2.5 0 180) (size 1.6 1.6) (drill 0.8) (layers *.Cu *.Mask) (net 81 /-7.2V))
  (pad 1 thru_hole rect (at 0 0 180) (size 1.6 1.6) (drill 0.8) (layers *.Cu *.Mask) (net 85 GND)))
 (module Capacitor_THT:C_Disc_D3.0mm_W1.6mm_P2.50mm (layer F.Cu) (at 132.715 113.07 270)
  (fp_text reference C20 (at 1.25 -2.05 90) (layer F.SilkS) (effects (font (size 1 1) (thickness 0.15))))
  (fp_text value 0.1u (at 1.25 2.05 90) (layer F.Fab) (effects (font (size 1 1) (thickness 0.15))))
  (pad 2 thru_hole circle (at 2.5 0 270) (size 1.6 1.6) (drill 0.8) (layers *.Cu *.Mask) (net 85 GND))
  (pad 1 thru_hole circle (at 0 0 270) (size 1.6 1.6) (drill 0.8) (layers *.Cu *.Mask) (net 84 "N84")))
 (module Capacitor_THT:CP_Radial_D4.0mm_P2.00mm (layer F.Cu) (at 170.18 111.76 90)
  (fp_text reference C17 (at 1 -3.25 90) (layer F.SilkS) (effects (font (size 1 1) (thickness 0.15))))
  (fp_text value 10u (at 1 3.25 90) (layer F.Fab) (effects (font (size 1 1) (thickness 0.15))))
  (pad 2 thru_hole circle (at 2 0 90) (size 1.2 1.2) (drill 0.6) (layers *.Cu *.Mask) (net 85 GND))
  (pad 1 thru_hole rect (at 0 0 90) (size 1.2 1.2) (drill 0.6) (layers *.Cu *.Mask) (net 104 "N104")))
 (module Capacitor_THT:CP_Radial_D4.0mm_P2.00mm (layer F.Cu) (at 160.02 101.6)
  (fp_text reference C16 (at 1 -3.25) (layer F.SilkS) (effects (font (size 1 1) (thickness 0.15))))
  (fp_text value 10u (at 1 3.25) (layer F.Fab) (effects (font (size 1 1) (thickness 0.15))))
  (pad 2 thru_hole circle (at 2 0) (size 1.2 1.2) (drill 0.6) (layers *.Cu *.Mask) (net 85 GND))
  (pad 1 thru_hole rect (at 0 0) (size 1.2 1.2) (drill 0.6) (layers *.Cu *.Mask) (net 103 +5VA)))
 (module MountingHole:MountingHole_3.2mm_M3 (layer F.Cu) (at 118.025 148.65)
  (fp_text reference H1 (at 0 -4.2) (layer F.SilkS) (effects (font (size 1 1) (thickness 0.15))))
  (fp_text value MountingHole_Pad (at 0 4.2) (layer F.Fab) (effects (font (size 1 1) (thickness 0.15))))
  (pad 1 thru_hole circle (at 0 0) (size 3.2 3.2) (drill 3.2) (layers *.Cu *.Mask) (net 85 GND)))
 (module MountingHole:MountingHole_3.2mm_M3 (layer F.Cu) (at 59.225 148.725)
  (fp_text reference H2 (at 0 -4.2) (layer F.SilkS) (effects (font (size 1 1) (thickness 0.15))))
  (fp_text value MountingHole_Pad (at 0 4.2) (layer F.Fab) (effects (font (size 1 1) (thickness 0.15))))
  (pad 1 thru_hole circle (at 0 0) (size 3.2 3.2) (drill 3.2) (layers *.Cu *.Mask) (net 85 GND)))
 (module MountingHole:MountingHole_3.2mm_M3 (layer F.Cu) (at 118.025 66.925)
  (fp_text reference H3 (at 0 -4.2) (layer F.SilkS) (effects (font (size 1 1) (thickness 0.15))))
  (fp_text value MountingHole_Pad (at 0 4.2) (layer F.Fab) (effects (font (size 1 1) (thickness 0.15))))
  (pad 1 thru_hole circle (at 0 0) (size 3.2 3.2) (drill 3.2) (layers *.Cu *.Mask) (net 85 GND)))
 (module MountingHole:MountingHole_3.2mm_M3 (layer F.Cu) (at 59.75 66.925)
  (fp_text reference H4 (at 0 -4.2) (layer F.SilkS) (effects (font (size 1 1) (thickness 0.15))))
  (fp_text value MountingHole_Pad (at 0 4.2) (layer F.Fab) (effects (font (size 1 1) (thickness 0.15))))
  (pad 1 thru_hole circle (at 0 0) (size 3.2 3.2) (drill 3.2) (layers *.Cu *.Mask) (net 85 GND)))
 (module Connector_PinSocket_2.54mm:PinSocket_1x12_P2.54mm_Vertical (layer F.Cu) (at 74.375 148.35 90)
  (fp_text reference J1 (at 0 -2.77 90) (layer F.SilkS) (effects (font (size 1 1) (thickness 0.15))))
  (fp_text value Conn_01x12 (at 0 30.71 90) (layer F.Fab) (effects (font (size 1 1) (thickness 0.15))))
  (pad 1 thru_hole rect (at 0 0 90) (size 1.7 1.7) (drill 1) (layers *.Cu *.Mask) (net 100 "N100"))
  (pad 2 thru_hole oval (at 0 2.54 90) (size 1.7 1.7) (drill 1) (layers *.Cu *.Mask) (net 87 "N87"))
  (pad 3 thru_hole oval (at 0 5.08 90) (size 1.7 1.7) (drill 1) (layers *.Cu *.Mask) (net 89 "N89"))
  (pad 4 thru_hole oval (at 0 7.62 90) (size 1.7 1.7) (drill 1) (layers *.Cu *.Mask) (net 90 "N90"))
  (pad 5 thru_hole oval (at 0 10.16 90) (size 1.7 1.7) (drill 1) (layers *.Cu *.Mask) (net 97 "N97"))
  (pad 6 thru_hole oval (at 0 12.7 90) (size 1.7 1.7) (drill 1) (layers *.Cu *.Mask) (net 99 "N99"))
  (pad 7 thru_hole oval (at 0 15.24 90) (size 1.7 1.7) (drill 1) (layers *.Cu *.Mask) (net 85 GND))
  (pad 8 thru_hole oval (at 0 17.78 90) (size 1.7 1.7) (drill 1) (layers *.Cu *.Mask) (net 85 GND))
  (pad 9 thru_hole oval (at 0 20.32 90) (size 1.7 1.7) (drill 1) (layers *.Cu *.Mask) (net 85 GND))
  (pad 10 thru_hole oval (at 0 22.86 90) (size 1.7 1.7) (drill 1) (layers *.Cu *.Mask) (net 104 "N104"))
  (pad 11 thru_hole oval (at 0 25.4 90) (size 1.7 1.7) (drill 1) (layers *.Cu *.Mask) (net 103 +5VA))
  (pad 12 thru_hole oval (at 0 27.94 90) (size 1.7 1.7) (drill 1) (layers *.Cu *.Mask) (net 81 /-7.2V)))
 (gr_line (start 55.725 152.425) (end 121.75 152.3) (layer Edge.Cuts) (width 0.05))
 (gr_line (start 55.825 63.475) (end 121.875 63.375) (layer Edge.Cuts) (width 0.05))
 (gr_line (start 55.88 63.5) (end 55.88 152.4) (layer Edge.Cuts) (width 0.05))
 (gr_line (start 121.925 152.4) (end 121.925 63.5) (layer Edge.Cuts) (width 0.05))
 (via (at 154.94 121.92) (size 0.8) (drill 0.4) (layers F.Cu B.Cu) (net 104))
 (via (at 154.94 127) (size 0.8) (drill 0.4) (layers F.Cu B.Cu) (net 104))
 (via (at 126.365 92.71) (size 0.8) (drill 0.4) (layers F.Cu B.Cu) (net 93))
 (via (at 126.365 75.565) (size 0.8) (drill 0.4) (layers F.Cu B.Cu) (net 93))
 (segment (start 102.235 92.71) (end 101.6 92.71) (width 1) (layer B.Cu) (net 95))
 (segment (start 97.79 79.375) (end 97.79 78.74) (width 1) (layer B.Cu) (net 102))
 (segment (start 145.335 77.47) (end 145.415 77.55) (width 2) (layer B.Cu) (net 85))
 (segment (start 162.56 102.14) (end 162.02 101.6) (width 2) (layer B.Cu) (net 85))
 (via (at 129.54 115.57) (size 0.8) (drill 0.4) (layers F.Cu B.Cu) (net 85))
 (via (at 114.3 115.57) (size 0.8) (drill 0.4) (layers F.Cu B.Cu) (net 85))
 (segment (start 114.3 115.57) (end 114.3 116.84) (width 2) (layer B.Cu) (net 85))
 (via (at 151.13 107.95) (size 0.8) (drill 0.4) (layers F.Cu B.Cu) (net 103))
 (via (at 151.13 128.27) (size 0.8) (drill 0.4) (layers F.Cu B.Cu) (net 103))
 (via (at 85.725 119.38) (size 0.8) (drill 0.4) (layers F.Cu B.Cu) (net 103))
 (via (at 116.205 119.38) (size 0.8) (drill 0.4) (layers F.Cu B.Cu) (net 103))
 (segment (start 137.63 88.9) (end 137.755 88.775) (width 0.25) (layer B.Cu) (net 81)))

